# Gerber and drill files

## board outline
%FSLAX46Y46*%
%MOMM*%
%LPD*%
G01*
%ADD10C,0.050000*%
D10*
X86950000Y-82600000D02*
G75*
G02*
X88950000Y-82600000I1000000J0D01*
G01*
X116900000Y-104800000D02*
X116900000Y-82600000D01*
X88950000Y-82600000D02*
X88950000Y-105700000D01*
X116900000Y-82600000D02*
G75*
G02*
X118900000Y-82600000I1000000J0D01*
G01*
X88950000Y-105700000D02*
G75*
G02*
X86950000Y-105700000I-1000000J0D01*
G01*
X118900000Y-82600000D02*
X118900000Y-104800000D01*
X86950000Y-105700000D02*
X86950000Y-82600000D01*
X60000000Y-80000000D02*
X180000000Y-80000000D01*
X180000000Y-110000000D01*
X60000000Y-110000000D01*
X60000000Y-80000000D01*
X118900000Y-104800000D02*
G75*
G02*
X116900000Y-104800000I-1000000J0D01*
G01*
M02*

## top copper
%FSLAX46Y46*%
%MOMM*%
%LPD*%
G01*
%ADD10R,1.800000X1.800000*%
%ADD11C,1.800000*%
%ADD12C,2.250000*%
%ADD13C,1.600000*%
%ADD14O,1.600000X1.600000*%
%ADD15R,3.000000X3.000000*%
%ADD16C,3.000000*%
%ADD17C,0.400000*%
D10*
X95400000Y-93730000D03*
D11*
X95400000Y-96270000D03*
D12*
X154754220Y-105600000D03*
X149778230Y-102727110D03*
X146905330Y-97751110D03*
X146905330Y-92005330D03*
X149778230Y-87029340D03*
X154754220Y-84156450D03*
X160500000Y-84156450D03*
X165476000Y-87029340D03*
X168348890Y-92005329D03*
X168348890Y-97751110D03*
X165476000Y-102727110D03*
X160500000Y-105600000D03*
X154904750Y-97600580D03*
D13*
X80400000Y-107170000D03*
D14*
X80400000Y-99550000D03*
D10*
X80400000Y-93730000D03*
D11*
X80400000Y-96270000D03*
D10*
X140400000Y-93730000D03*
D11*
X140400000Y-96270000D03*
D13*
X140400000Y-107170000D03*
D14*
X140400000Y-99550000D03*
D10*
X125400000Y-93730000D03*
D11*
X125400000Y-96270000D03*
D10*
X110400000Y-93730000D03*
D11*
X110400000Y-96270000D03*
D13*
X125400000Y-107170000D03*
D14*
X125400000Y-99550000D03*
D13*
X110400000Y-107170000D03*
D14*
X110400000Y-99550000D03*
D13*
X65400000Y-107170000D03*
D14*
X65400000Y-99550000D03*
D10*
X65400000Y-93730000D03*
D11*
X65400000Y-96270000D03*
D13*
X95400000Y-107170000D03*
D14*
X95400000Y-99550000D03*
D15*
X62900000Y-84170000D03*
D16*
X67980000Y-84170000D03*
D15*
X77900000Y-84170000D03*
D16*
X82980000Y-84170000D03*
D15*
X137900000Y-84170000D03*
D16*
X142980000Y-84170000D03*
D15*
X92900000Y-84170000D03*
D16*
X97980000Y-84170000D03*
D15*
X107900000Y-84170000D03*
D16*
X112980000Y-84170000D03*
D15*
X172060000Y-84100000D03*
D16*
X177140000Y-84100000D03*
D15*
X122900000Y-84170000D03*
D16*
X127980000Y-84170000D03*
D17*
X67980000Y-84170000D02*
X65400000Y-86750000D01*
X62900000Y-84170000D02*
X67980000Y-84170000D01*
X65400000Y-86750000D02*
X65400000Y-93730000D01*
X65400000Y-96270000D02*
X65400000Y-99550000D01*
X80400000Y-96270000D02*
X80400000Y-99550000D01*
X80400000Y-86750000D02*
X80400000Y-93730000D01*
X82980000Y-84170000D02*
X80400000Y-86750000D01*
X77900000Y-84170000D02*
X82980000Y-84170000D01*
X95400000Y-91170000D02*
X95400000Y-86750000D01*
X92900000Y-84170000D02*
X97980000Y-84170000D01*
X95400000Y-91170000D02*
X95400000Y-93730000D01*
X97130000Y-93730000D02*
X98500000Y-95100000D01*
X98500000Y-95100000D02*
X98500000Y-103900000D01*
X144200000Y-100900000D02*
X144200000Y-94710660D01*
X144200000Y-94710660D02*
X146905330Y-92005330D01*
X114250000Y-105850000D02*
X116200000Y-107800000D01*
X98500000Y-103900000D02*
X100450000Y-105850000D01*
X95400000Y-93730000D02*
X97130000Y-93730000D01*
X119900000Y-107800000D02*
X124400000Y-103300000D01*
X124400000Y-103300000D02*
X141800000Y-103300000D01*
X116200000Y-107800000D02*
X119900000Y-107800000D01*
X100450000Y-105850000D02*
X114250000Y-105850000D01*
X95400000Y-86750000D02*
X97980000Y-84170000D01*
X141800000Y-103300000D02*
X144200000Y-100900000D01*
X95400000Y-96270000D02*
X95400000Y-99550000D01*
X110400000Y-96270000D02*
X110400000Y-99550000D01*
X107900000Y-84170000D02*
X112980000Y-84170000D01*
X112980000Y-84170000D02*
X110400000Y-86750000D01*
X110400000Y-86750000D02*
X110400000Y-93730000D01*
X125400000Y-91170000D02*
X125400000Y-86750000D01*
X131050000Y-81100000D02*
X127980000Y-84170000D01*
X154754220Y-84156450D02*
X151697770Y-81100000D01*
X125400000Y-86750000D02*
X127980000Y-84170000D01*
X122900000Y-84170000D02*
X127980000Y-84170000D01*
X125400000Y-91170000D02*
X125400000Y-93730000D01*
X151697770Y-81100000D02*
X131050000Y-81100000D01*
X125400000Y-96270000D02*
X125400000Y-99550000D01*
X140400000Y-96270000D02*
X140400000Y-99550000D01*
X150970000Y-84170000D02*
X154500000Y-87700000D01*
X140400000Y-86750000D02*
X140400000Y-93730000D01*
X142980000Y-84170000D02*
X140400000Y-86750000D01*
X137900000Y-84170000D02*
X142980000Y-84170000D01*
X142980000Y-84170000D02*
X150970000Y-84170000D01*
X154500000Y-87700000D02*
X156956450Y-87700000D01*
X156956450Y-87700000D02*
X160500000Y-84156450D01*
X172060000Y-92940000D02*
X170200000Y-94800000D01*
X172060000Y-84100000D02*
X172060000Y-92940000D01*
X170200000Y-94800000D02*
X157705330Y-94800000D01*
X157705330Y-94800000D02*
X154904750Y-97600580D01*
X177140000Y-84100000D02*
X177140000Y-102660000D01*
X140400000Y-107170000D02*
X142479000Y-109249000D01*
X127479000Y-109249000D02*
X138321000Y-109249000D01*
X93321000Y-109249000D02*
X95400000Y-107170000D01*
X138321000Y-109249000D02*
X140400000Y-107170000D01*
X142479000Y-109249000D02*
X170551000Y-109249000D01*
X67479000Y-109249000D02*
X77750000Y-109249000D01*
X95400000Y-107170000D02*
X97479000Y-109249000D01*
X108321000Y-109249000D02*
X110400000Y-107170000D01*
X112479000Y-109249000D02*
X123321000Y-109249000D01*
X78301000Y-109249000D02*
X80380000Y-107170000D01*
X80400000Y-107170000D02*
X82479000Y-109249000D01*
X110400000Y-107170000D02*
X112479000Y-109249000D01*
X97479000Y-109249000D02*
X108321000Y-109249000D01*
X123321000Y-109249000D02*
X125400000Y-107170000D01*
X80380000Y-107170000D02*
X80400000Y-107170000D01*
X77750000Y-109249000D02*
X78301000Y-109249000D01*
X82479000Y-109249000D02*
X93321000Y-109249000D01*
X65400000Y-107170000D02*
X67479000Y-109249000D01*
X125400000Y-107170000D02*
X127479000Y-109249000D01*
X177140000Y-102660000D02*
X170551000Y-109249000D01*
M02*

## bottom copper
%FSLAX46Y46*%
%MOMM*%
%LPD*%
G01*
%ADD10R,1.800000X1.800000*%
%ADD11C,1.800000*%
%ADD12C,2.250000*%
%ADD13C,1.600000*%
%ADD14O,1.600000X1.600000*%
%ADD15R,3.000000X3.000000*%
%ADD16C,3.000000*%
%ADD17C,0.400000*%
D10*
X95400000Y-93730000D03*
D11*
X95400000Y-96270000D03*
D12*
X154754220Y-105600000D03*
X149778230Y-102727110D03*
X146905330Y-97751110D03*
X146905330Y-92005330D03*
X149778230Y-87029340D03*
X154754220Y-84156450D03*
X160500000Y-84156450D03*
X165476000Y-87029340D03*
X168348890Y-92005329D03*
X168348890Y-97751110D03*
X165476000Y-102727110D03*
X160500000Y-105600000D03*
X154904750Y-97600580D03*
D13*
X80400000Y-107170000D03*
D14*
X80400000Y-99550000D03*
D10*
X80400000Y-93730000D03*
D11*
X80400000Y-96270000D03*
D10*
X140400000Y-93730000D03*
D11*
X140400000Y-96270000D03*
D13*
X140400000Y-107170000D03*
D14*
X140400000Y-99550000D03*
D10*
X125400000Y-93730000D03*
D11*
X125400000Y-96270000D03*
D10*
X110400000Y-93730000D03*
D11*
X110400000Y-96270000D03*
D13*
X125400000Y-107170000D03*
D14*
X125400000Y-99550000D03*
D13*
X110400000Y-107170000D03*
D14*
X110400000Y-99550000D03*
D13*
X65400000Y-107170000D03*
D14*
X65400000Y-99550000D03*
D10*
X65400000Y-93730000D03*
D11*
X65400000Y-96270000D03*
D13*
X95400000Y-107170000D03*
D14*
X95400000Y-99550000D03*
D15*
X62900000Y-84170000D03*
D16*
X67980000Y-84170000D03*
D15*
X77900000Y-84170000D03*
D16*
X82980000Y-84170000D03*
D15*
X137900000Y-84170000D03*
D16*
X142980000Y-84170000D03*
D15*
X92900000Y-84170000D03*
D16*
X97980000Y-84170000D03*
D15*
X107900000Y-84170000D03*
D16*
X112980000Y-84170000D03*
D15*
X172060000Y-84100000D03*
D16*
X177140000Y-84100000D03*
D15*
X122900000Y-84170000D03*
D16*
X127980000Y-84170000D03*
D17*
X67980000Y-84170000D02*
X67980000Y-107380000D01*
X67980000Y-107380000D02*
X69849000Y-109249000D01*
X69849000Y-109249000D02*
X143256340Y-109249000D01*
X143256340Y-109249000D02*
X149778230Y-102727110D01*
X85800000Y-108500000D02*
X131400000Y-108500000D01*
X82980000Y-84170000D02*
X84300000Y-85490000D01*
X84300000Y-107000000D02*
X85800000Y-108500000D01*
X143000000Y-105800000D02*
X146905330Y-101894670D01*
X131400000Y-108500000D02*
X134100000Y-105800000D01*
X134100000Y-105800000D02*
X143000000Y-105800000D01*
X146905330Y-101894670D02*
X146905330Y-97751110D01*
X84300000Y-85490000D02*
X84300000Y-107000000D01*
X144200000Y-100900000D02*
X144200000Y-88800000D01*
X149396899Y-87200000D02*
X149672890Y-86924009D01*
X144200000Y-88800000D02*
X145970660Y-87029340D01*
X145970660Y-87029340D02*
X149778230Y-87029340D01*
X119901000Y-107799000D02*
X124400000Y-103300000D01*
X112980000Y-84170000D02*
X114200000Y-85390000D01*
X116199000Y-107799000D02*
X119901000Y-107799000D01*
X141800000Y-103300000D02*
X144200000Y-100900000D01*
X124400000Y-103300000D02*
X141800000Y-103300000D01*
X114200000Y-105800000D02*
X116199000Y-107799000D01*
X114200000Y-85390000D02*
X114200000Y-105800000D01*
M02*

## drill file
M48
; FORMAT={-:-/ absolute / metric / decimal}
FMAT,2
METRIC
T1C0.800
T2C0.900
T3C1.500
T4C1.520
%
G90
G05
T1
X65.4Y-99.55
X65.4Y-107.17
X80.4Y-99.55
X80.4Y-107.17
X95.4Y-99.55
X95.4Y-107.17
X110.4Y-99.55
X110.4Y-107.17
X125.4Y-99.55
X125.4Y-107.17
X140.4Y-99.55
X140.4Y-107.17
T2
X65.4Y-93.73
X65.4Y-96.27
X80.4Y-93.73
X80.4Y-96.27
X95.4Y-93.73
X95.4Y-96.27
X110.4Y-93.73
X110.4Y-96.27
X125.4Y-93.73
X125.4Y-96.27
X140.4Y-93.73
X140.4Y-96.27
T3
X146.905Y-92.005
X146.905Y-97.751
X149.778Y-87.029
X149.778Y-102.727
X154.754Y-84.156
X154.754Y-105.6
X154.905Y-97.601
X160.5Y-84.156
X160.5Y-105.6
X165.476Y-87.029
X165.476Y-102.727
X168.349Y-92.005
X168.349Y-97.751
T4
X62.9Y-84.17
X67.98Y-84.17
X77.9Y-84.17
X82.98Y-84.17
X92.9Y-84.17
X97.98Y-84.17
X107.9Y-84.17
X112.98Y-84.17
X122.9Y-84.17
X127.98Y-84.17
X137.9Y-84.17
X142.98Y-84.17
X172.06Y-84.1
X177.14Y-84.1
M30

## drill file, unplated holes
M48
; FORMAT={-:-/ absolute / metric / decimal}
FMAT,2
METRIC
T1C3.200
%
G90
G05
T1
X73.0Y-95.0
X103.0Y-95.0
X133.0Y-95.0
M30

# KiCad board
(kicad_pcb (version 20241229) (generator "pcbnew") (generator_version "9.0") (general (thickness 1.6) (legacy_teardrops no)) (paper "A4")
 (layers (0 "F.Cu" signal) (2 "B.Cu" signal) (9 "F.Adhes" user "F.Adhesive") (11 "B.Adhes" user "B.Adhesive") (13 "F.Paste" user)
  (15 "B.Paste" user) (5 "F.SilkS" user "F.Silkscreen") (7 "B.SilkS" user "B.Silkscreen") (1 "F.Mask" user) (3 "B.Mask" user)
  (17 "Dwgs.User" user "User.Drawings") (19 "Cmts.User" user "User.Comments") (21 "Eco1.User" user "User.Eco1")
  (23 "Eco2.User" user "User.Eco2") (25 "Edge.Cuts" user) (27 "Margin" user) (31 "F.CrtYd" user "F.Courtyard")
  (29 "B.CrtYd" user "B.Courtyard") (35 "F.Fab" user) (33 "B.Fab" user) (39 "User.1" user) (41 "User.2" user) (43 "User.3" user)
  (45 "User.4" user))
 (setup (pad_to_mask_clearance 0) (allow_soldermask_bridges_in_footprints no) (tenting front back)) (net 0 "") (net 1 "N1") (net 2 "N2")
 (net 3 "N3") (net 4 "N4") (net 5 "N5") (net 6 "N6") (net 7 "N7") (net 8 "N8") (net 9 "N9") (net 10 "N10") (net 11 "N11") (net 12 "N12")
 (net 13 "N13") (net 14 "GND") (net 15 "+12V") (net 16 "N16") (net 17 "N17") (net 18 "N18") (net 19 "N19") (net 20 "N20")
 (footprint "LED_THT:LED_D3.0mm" (layer "F.Cu") (at 95.4 93.73 -90)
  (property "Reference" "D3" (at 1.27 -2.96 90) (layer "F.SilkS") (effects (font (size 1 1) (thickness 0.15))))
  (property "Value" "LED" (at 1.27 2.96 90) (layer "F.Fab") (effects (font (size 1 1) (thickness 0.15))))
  (pad "1" thru_hole rect (at 0 0 270) (size 1.8 1.8) (drill 0.9) (layers "*.Cu" "*.Mask") (remove_unused_layers no) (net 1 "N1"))
  (pad "2" thru_hole circle (at 2.54 0 270) (size 1.8 1.8) (drill 0.9) (layers "*.Cu" "*.Mask") (remove_unused_layers no) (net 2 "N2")))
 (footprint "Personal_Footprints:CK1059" (layer "F.Cu") (at 154.75422 105.6)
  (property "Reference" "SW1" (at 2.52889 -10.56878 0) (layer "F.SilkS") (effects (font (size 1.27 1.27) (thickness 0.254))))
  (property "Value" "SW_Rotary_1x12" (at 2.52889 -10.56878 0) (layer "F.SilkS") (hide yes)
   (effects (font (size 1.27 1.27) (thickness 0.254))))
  (pad "1" thru_hole circle (at 0 0) (size 2.25 2.25) (drill 1.5) (layers "*.Cu" "*.Mask") (remove_unused_layers no) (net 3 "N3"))
  (pad "2" thru_hole circle (at -4.97599 -2.87289) (size 2.25 2.25) (drill 1.5) (layers "*.Cu" "*.Mask") (remove_unused_layers no)
   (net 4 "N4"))
  (pad "3" thru_hole circle (at -7.84889 -7.84889) (size 2.25 2.25) (drill 1.5) (layers "*.Cu" "*.Mask") (remove_unused_layers no)
   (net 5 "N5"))
  (pad "4" thru_hole circle (at -7.84889 -13.59467) (size 2.25 2.25) (drill 1.5) (layers "*.Cu" "*.Mask") (remove_unused_layers no)
   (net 1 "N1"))
  (pad "5" thru_hole circle (at -4.97599 -18.57066) (size 2.25 2.25) (drill 1.5) (layers "*.Cu" "*.Mask") (remove_unused_layers no)
   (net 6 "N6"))
  (pad "6" thru_hole circle (at 0 -21.44355) (size 2.25 2.25) (drill 1.5) (layers "*.Cu" "*.Mask") (remove_unused_layers no) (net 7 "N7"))
  (pad "7" thru_hole circle (at 5.74578 -21.44355) (size 2.25 2.25) (drill 1.5) (layers "*.Cu" "*.Mask") (remove_unused_layers no)
   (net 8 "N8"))
  (pad "8" thru_hole circle (at 10.72178 -18.57066) (size 2.25 2.25) (drill 1.5) (layers "*.Cu" "*.Mask") (remove_unused_layers no)
   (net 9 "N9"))
  (pad "9" thru_hole circle (at 13.59467 -13.594671) (size 2.25 2.25) (drill 1.5) (layers "*.Cu" "*.Mask") (remove_unused_layers no)
   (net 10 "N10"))
  (pad "10" thru_hole circle (at 13.59467 -7.84889) (size 2.25 2.25) (drill 1.5) (layers "*.Cu" "*.Mask") (remove_unused_layers no)
   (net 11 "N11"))
  (pad "11" thru_hole circle (at 10.72178 -2.87289) (size 2.25 2.25) (drill 1.5) (layers "*.Cu" "*.Mask") (remove_unused_layers no)
   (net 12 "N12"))
  (pad "12" thru_hole circle (at 5.74578 0) (size 2.25 2.25) (drill 1.5) (layers "*.Cu" "*.Mask") (remove_unused_layers no) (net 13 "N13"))
  (pad "13" thru_hole circle (at 0.15053 -7.99942) (size 2.25 2.25) (drill 1.5) (layers "*.Cu" "*.Mask") (remove_unused_layers no)
   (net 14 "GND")))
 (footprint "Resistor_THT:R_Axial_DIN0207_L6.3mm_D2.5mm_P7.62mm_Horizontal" (layer "F.Cu") (at 80.4 107.17 90)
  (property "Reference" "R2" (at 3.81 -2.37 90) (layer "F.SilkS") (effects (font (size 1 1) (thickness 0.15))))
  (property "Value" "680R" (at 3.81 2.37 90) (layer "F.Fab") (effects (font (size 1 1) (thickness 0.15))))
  (pad "1" thru_hole circle (at 0 0 90) (size 1.6 1.6) (drill 0.8) (layers "*.Cu" "*.Mask") (remove_unused_layers no) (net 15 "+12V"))
  (pad "2" thru_hole oval (at 7.62 0 90) (size 1.6 1.6) (drill 0.8) (layers "*.Cu" "*.Mask") (remove_unused_layers no) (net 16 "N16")))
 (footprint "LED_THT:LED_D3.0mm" (layer "F.Cu") (at 80.4 93.73 -90)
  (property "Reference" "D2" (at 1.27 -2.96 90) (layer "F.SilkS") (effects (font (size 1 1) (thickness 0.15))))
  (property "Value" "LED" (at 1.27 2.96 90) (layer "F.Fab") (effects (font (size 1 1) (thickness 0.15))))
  (pad "1" thru_hole rect (at 0 0 270) (size 1.8 1.8) (drill 0.9) (layers "*.Cu" "*.Mask") (remove_unused_layers no) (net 5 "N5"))
  (pad "2" thru_hole circle (at 2.54 0 270) (size 1.8 1.8) (drill 0.9) (layers "*.Cu" "*.Mask") (remove_unused_layers no) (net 16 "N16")))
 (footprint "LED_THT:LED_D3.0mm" (layer "F.Cu") (at 140.4 93.73 -90)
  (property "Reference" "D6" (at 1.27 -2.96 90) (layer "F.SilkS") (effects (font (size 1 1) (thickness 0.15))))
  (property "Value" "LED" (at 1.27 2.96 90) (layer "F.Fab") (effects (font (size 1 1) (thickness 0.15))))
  (pad "1" thru_hole rect (at 0 0 270) (size 1.8 1.8) (drill 0.9) (layers "*.Cu" "*.Mask") (remove_unused_layers no) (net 8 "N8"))
  (pad "2" thru_hole circle (at 2.54 0 270) (size 1.8 1.8) (drill 0.9) (layers "*.Cu" "*.Mask") (remove_unused_layers no) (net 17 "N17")))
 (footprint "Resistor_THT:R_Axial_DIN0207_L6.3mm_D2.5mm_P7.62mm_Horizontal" (layer "F.Cu") (at 140.4 107.17 90)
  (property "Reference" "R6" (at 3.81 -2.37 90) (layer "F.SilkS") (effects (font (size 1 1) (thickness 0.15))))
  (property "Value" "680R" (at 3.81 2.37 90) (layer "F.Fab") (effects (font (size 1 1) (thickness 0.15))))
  (pad "1" thru_hole circle (at 0 0 90) (size 1.6 1.6) (drill 0.8) (layers "*.Cu" "*.Mask") (remove_unused_layers no) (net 15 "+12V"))
  (pad "2" thru_hole oval (at 7.62 0 90) (size 1.6 1.6) (drill 0.8) (layers "*.Cu" "*.Mask") (remove_unused_layers no) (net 17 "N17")))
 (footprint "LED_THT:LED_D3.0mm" (layer "F.Cu") (at 125.4 93.73 -90)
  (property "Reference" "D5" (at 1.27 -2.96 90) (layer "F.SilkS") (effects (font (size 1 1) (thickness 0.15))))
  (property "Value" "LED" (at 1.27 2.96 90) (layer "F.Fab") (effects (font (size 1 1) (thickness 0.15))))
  (pad "1" thru_hole rect (at 0 0 270) (size 1.8 1.8) (drill 0.9) (layers "*.Cu" "*.Mask") (remove_unused_layers no) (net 7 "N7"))
  (pad "2" thru_hole circle (at 2.54 0 270) (size 1.8 1.8) (drill 0.9) (layers "*.Cu" "*.Mask") (remove_unused_layers no) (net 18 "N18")))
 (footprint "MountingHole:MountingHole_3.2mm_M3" (layer "F.Cu") (at 103 95)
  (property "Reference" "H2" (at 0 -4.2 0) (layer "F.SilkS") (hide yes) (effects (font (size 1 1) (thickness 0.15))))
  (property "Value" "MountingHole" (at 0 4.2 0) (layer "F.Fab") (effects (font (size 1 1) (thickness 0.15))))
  (pad "" np_thru_hole circle (at 0 0) (size 3.2 3.2) (drill 3.2) (layers "*.Cu" "*.Mask")))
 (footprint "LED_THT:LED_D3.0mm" (layer "F.Cu") (at 110.4 93.73 -90)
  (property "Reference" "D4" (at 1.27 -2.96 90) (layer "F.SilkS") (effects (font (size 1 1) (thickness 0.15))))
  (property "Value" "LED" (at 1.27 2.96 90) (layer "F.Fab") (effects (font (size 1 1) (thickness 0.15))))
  (pad "1" thru_hole rect (at 0 0 270) (size 1.8 1.8) (drill 0.9) (layers "*.Cu" "*.Mask") (remove_unused_layers no) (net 6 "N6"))
  (pad "2" thru_hole circle (at 2.54 0 270) (size 1.8 1.8) (drill 0.9) (layers "*.Cu" "*.Mask") (remove_unused_layers no) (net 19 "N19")))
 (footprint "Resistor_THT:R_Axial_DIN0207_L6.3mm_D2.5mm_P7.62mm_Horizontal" (layer "F.Cu") (at 125.4 107.17 90)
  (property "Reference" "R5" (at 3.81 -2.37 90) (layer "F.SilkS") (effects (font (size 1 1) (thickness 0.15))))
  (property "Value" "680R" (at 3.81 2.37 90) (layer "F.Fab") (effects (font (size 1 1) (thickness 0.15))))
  (pad "1" thru_hole circle (at 0 0 90) (size 1.6 1.6) (drill 0.8) (layers "*.Cu" "*.Mask") (remove_unused_layers no) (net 15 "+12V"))
  (pad "2" thru_hole oval (at 7.62 0 90) (size 1.6 1.6) (drill 0.8) (layers "*.Cu" "*.Mask") (remove_unused_layers no) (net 18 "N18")))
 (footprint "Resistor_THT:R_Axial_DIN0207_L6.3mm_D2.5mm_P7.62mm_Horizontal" (layer "F.Cu") (at 110.4 107.17 90)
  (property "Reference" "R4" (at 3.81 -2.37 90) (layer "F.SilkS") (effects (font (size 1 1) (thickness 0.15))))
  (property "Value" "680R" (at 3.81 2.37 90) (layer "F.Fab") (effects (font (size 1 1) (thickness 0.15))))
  (pad "1" thru_hole circle (at 0 0 90) (size 1.6 1.6) (drill 0.8) (layers "*.Cu" "*.Mask") (remove_unused_layers no) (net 15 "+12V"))
  (pad "2" thru_hole oval (at 7.62 0 90) (size 1.6 1.6) (drill 0.8) (layers "*.Cu" "*.Mask") (remove_unused_layers no) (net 19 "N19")))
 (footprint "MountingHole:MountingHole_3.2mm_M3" (layer "F.Cu") (at 73 95)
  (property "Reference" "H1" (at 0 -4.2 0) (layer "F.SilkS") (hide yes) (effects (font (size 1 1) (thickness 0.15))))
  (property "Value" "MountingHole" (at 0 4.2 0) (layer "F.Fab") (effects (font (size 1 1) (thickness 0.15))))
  (pad "" np_thru_hole circle (at 0 0) (size 3.2 3.2) (drill 3.2) (layers "*.Cu" "*.Mask")))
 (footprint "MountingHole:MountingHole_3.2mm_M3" (layer "F.Cu") (at 133 95)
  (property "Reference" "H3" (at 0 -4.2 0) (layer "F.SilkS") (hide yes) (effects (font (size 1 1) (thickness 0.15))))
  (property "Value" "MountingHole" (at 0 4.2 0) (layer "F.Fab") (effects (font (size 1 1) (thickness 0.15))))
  (pad "" np_thru_hole circle (at 0 0) (size 3.2 3.2) (drill 3.2) (layers "*.Cu" "*.Mask")))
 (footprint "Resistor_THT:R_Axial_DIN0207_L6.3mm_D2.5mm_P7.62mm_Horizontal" (layer "F.Cu") (at 65.4 107.17 90)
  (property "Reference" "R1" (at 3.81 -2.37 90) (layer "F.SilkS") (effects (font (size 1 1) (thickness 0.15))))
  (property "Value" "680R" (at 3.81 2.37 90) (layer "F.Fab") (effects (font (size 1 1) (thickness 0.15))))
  (pad "1" thru_hole circle (at 0 0 90) (size 1.6 1.6) (drill 0.8) (layers "*.Cu" "*.Mask") (remove_unused_layers no) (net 15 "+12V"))
  (pad "2" thru_hole oval (at 7.62 0 90) (size 1.6 1.6) (drill 0.8) (layers "*.Cu" "*.Mask") (remove_unused_layers no) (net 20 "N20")))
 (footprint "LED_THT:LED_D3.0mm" (layer "F.Cu") (at 65.4 93.73 -90)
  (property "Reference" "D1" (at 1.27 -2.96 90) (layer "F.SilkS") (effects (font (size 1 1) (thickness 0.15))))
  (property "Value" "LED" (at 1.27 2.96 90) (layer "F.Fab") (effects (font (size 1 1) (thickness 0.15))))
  (pad "1" thru_hole rect (at 0 0 270) (size 1.8 1.8) (drill 0.9) (layers "*.Cu" "*.Mask") (remove_unused_layers no) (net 4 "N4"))
  (pad "2" thru_hole circle (at 2.54 0 270) (size 1.8 1.8) (drill 0.9) (layers "*.Cu" "*.Mask") (remove_unused_layers no) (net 20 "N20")))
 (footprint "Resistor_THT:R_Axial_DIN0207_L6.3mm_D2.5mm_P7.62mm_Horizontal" (layer "F.Cu") (at 95.4 107.17 90)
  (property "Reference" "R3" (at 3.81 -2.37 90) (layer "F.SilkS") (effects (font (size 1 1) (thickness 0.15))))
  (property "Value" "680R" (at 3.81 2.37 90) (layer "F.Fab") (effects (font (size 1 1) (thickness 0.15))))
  (pad "1" thru_hole circle (at 0 0 90) (size 1.6 1.6) (drill 0.8) (layers "*.Cu" "*.Mask") (remove_unused_layers no) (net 15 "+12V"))
  (pad "2" thru_hole oval (at 7.62 0 90) (size 1.6 1.6) (drill 0.8) (layers "*.Cu" "*.Mask") (remove_unused_layers no) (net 2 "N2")))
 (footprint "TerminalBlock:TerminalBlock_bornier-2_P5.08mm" (layer "B.Cu") (at 62.9 84.17)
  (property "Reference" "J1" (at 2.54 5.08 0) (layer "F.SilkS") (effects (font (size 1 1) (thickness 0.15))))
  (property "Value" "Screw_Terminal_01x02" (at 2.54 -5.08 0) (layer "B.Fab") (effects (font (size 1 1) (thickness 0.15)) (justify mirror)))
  (pad "1" thru_hole rect (at 0 0) (size 3 3) (drill 1.52) (layers "*.Cu" "*.Mask") (remove_unused_layers no) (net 4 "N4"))
  (pad "2" thru_hole circle (at 5.08 0) (size 3 3) (drill 1.52) (layers "*.Cu" "*.Mask") (remove_unused_layers no) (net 4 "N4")))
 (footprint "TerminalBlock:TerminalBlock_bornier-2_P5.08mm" (layer "B.Cu") (at 77.9 84.17)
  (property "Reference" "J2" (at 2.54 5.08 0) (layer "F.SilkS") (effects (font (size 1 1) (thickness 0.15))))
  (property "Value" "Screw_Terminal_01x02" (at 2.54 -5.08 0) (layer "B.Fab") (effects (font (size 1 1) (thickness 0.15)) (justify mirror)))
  (pad "1" thru_hole rect (at 0 0) (size 3 3) (drill 1.52) (layers "*.Cu" "*.Mask") (remove_unused_layers no) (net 5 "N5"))
  (pad "2" thru_hole circle (at 5.08 0) (size 3 3) (drill 1.52) (layers "*.Cu" "*.Mask") (remove_unused_layers no) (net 5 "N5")))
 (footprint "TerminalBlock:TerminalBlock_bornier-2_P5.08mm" (layer "B.Cu") (at 137.9 84.17)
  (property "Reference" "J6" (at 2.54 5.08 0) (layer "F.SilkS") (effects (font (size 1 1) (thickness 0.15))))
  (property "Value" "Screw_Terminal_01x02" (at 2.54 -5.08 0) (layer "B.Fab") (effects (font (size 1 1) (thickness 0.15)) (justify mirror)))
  (pad "1" thru_hole rect (at 0 0) (size 3 3) (drill 1.52) (layers "*.Cu" "*.Mask") (remove_unused_layers no) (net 8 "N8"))
  (pad "2" thru_hole circle (at 5.08 0) (size 3 3) (drill 1.52) (layers "*.Cu" "*.Mask") (remove_unused_layers no) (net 8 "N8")))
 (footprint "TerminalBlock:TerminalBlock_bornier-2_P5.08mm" (layer "B.Cu") (at 92.9 84.17)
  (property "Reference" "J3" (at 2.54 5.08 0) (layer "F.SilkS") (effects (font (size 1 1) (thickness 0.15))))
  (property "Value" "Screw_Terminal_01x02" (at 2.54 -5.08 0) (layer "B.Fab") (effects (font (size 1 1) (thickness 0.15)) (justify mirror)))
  (pad "1" thru_hole rect (at 0 0) (size 3 3) (drill 1.52) (layers "*.Cu" "*.Mask") (remove_unused_layers no) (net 1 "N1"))
  (pad "2" thru_hole circle (at 5.08 0) (size 3 3) (drill 1.52) (layers "*.Cu" "*.Mask") (remove_unused_layers no) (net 1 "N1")))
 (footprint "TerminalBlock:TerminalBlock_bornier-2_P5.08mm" (layer "B.Cu") (at 107.9 84.17)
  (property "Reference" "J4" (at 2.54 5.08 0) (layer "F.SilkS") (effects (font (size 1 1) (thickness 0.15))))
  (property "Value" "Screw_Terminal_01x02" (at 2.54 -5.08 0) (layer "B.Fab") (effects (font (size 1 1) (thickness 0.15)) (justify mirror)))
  (pad "1" thru_hole rect (at 0 0) (size 3 3) (drill 1.52) (layers "*.Cu" "*.Mask") (remove_unused_layers no) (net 6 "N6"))
  (pad "2" thru_hole circle (at 5.08 0) (size 3 3) (drill 1.52) (layers "*.Cu" "*.Mask") (remove_unused_layers no) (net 6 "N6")))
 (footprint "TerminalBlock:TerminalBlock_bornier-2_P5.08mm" (layer "B.Cu") (at 172.06 84.1)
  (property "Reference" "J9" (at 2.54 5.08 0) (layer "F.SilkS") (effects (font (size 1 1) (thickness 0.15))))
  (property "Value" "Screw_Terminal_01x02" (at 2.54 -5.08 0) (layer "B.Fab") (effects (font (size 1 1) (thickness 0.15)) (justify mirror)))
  (pad "1" thru_hole rect (at 0 0) (size 3 3) (drill 1.52) (layers "*.Cu" "*.Mask") (remove_unused_layers no) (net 14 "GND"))
  (pad "2" thru_hole circle (at 5.08 0) (size 3 3) (drill 1.52) (layers "*.Cu" "*.Mask") (remove_unused_layers no) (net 15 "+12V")))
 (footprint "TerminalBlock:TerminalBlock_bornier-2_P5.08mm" (layer "B.Cu") (at 122.9 84.17)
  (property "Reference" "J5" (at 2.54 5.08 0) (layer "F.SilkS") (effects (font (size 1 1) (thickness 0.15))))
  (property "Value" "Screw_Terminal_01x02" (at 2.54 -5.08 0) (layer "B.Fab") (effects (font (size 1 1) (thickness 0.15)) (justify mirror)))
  (pad "1" thru_hole rect (at 0 0) (size 3 3) (drill 1.52) (layers "*.Cu" "*.Mask") (remove_unused_layers no) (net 7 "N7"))
  (pad "2" thru_hole circle (at 5.08 0) (size 3 3) (drill 1.52) (layers "*.Cu" "*.Mask") (remove_unused_layers no) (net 7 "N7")))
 (gr_arc (start 86.95 82.6) (mid 87.95 81.6) (end 88.95 82.6) (stroke (width 0.05) (type default)) (layer "Edge.Cuts"))
 (gr_line (start 116.9 104.8) (end 116.9 82.6) (stroke (width 0.05) (type default)) (layer "Edge.Cuts"))
 (gr_line (start 88.95 82.6) (end 88.95 105.7) (stroke (width 0.05) (type default)) (layer "Edge.Cuts"))
 (gr_arc (start 116.9 82.6) (mid 117.9 81.6) (end 118.9 82.6) (stroke (width 0.05) (type default)) (layer "Edge.Cuts"))
 (gr_arc (start 88.95 105.7) (mid 87.95 106.7) (end 86.95 105.7) (stroke (width 0.05) (type default)) (layer "Edge.Cuts"))
 (gr_line (start 118.9 82.6) (end 118.9 104.8) (stroke (width 0.05) (type default)) (layer "Edge.Cuts"))
 (gr_line (start 86.95 105.7) (end 86.95 82.6) (stroke (width 0.05) (type default)) (layer "Edge.Cuts"))
 (gr_rect (start 60 80) (end 180 110) (stroke (width 0.05) (type solid)) (fill no) (layer "Edge.Cuts"))
 (gr_arc (start 118.9 104.8) (mid 117.9 105.8) (end 116.9 104.8) (stroke (width 0.05) (type default)) (layer "Edge.Cuts"))
 (segment (start 67.98 84.17) (end 65.4 86.75) (width 0.4) (layer "F.Cu") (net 4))
 (segment (start 62.9 84.17) (end 67.98 84.17) (width 0.4) (layer "F.Cu") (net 4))
 (segment (start 65.4 86.75) (end 65.4 93.73) (width 0.4) (layer "F.Cu") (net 4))
 (segment (start 67.98 84.17) (end 67.98 107.38) (width 0.4) (layer "B.Cu") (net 4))
 (segment (start 67.98 107.38) (end 69.849 109.249) (width 0.4) (layer "B.Cu") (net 4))
 (segment (start 69.849 109.249) (end 143.25634 109.249) (width 0.4) (layer "B.Cu") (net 4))
 (segment (start 143.25634 109.249) (end 149.77823 102.72711) (width 0.4) (layer "B.Cu") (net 4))
 (segment (start 65.4 96.27) (end 65.4 99.55) (width 0.4) (layer "F.Cu") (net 20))
 (segment (start 80.4 96.27) (end 80.4 99.55) (width 0.4) (layer "F.Cu") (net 16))
 (segment (start 80.4 86.75) (end 80.4 93.73) (width 0.4) (layer "F.Cu") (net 5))
 (segment (start 82.98 84.17) (end 80.4 86.75) (width 0.4) (layer "F.Cu") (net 5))
 (segment (start 77.9 84.17) (end 82.98 84.17) (width 0.4) (layer "F.Cu") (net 5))
 (segment (start 85.8 108.5) (end 131.4 108.5) (width 0.4) (layer "B.Cu") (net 5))
 (segment (start 82.98 84.17) (end 84.3 85.49) (width 0.4) (layer "B.Cu") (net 5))
 (segment (start 84.3 107) (end 85.8 108.5) (width 0.4) (layer "B.Cu") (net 5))
 (segment (start 143 105.8) (end 146.90533 101.89467) (width 0.4) (layer "B.Cu") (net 5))
 (segment (start 131.4 108.5) (end 134.1 105.8) (width 0.4) (layer "B.Cu") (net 5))
 (segment (start 134.1 105.8) (end 143 105.8) (width 0.4) (layer "B.Cu") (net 5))
 (segment (start 146.90533 101.89467) (end 146.90533 97.75111) (width 0.4) (layer "B.Cu") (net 5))
 (segment (start 84.3 85.49) (end 84.3 107) (width 0.4) (layer "B.Cu") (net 5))
 (segment (start 95.4 91.17) (end 95.4 86.75) (width 0.4) (layer "F.Cu") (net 1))
 (segment (start 92.9 84.17) (end 97.98 84.17) (width 0.4) (layer "F.Cu") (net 1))
 (segment (start 95.4 91.17) (end 95.4 93.73) (width 0.4) (layer "F.Cu") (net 1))
 (segment (start 97.13 93.73) (end 98.5 95.1) (width 0.4) (layer "F.Cu") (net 1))
 (segment (start 98.5 95.1) (end 98.5 103.9) (width 0.4) (layer "F.Cu") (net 1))
 (segment (start 144.2 100.9) (end 144.2 94.71066) (width 0.4) (layer "F.Cu") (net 1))
 (segment (start 144.2 94.71066) (end 146.90533 92.00533) (width 0.4) (layer "F.Cu") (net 1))
 (segment (start 114.25 105.85) (end 116.2 107.8) (width 0.4) (layer "F.Cu") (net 1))
 (segment (start 98.5 103.9) (end 100.45 105.85) (width 0.4) (layer "F.Cu") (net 1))
 (segment (start 95.4 93.73) (end 97.13 93.73) (width 0.4) (layer "F.Cu") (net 1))
 (segment (start 119.9 107.8) (end 124.4 103.3) (width 0.4) (layer "F.Cu") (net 1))
 (segment (start 124.4 103.3) (end 141.8 103.3) (width 0.4) (layer "F.Cu") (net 1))
 (segment (start 116.2 107.8) (end 119.9 107.8) (width 0.4) (layer "F.Cu") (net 1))
 (segment (start 100.45 105.85) (end 114.25 105.85) (width 0.4) (layer "F.Cu") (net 1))
 (segment (start 95.4 86.75) (end 97.98 84.17) (width 0.4) (layer "F.Cu") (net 1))
 (segment (start 141.8 103.3) (end 144.2 100.9) (width 0.4) (layer "F.Cu") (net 1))
 (segment (start 95.4 96.27) (end 95.4 99.55) (width 0.4) (layer "F.Cu") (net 2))
 (segment (start 110.4 96.27) (end 110.4 99.55) (width 0.4) (layer "F.Cu") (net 19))
 (segment (start 107.9 84.17) (end 112.98 84.17) (width 0.4) (layer "F.Cu") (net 6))
 (segment (start 112.98 84.17) (end 110.4 86.75) (width 0.4) (layer "F.Cu") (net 6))
 (segment (start 110.4 86.75) (end 110.4 93.73) (width 0.4) (layer "F.Cu") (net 6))
 (segment (start 144.2 100.9) (end 144.2 88.8) (width 0.4) (layer "B.Cu") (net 6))
 (segment (start 149.396899 87.2) (end 149.67289 86.924009) (width 0.4) (layer "B.Cu") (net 6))
 (segment (start 144.2 88.8) (end 145.97066 87.02934) (width 0.4) (layer "B.Cu") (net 6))
 (segment (start 145.97066 87.02934) (end 149.77823 87.02934) (width 0.4) (layer "B.Cu") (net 6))
 (segment (start 119.901 107.799) (end 124.4 103.3) (width 0.4) (layer "B.Cu") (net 6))
 (segment (start 112.98 84.17) (end 114.2 85.39) (width 0.4) (layer "B.Cu") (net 6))
 (segment (start 116.199 107.799) (end 119.901 107.799) (width 0.4) (layer "B.Cu") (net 6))
 (segment (start 141.8 103.3) (end 144.2 100.9) (width 0.4) (layer "B.Cu") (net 6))
 (segment (start 124.4 103.3) (end 141.8 103.3) (width 0.4) (layer "B.Cu") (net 6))
 (segment (start 114.2 105.8) (end 116.199 107.799) (width 0.4) (layer "B.Cu") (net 6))
 (segment (start 114.2 85.39) (end 114.2 105.8) (width 0.4) (layer "B.Cu") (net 6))
 (segment (start 125.4 91.17) (end 125.4 86.75) (width 0.4) (layer "F.Cu") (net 7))
 (segment (start 131.05 81.1) (end 127.98 84.17) (width 0.4) (layer "F.Cu") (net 7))
 (segment (start 154.75422 84.15645) (end 151.69777 81.1) (width 0.4) (layer "F.Cu") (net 7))
 (segment (start 125.4 86.75) (end 127.98 84.17) (width 0.4) (layer "F.Cu") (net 7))
 (segment (start 122.9 84.17) (end 127.98 84.17) (width 0.4) (layer "F.Cu") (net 7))
 (segment (start 125.4 91.17) (end 125.4 93.73) (width 0.4) (layer "F.Cu") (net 7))
 (segment (start 151.69777 81.1) (end 131.05 81.1) (width 0.4) (layer "F.Cu") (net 7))
 (segment (start 125.4 96.27) (end 125.4 99.55) (width 0.4) (layer "F.Cu") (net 18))
 (segment (start 140.4 96.27) (end 140.4 99.55) (width 0.4) (layer "F.Cu") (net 17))
 (segment (start 150.97 84.17) (end 154.5 87.7) (width 0.4) (layer "F.Cu") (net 8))
 (segment (start 140.4 86.75) (end 140.4 93.73) (width 0.4) (layer "F.Cu") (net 8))
 (segment (start 142.98 84.17) (end 140.4 86.75) (width 0.4) (layer "F.Cu") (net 8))
 (segment (start 137.9 84.17) (end 142.98 84.17) (width 0.4) (layer "F.Cu") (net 8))
 (segment (start 142.98 84.17) (end 150.97 84.17) (width 0.4) (layer "F.Cu") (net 8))
 (segment (start 154.5 87.7) (end 156.95645 87.7) (width 0.4) (layer "F.Cu") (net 8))
 (segment (start 156.95645 87.7) (end 160.5 84.15645) (width 0.4) (layer "F.Cu") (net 8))
 (segment (start 172.06 92.94) (end 170.2 94.8) (width 0.4) (layer "F.Cu") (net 14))
 (segment (start 172.06 84.1) (end 172.06 92.94) (width 0.4) (layer "F.Cu") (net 14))
 (segment (start 170.2 94.8) (end 157.70533 94.8) (width 0.4) (layer "F.Cu") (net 14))
 (segment (start 157.70533 94.8) (end 154.90475 97.60058) (width 0.4) (layer "F.Cu") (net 14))
 (segment (start 177.14 84.1) (end 177.14 102.66) (width 0.4) (layer "F.Cu") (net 15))
 (segment (start 140.4 107.17) (end 142.479 109.249) (width 0.4) (layer "F.Cu") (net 15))
 (segment (start 127.479 109.249) (end 138.321 109.249) (width 0.4) (layer "F.Cu") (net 15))
 (segment (start 93.321 109.249) (end 95.4 107.17) (width 0.4) (layer "F.Cu") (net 15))
 (segment (start 138.321 109.249) (end 140.4 107.17) (width 0.4) (layer "F.Cu") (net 15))
 (segment (start 142.479 109.249) (end 170.551 109.249) (width 0.4) (layer "F.Cu") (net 15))
 (segment (start 67.479 109.249) (end 77.75 109.249) (width 0.4) (layer "F.Cu") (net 15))
 (segment (start 95.4 107.17) (end 97.479 109.249) (width 0.4) (layer "F.Cu") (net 15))
 (segment (start 108.321 109.249) (end 110.4 107.17) (width 0.4) (layer "F.Cu") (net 15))
 (segment (start 112.479 109.249) (end 123.321 109.249) (width 0.4) (layer "F.Cu") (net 15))
 (segment (start 78.301 109.249) (end 80.38 107.17) (width 0.4) (layer "F.Cu") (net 15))
 (segment (start 80.4 107.17) (end 82.479 109.249) (width 0.4) (layer "F.Cu") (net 15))
 (segment (start 110.4 107.17) (end 112.479 109.249) (width 0.4) (layer "F.Cu") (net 15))
 (segment (start 97.479 109.249) (end 108.321 109.249) (width 0.4) (layer "F.Cu") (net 15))
 (segment (start 123.321 109.249) (end 125.4 107.17) (width 0.4) (layer "F.Cu") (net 15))
 (segment (start 80.38 107.17) (end 80.4 107.17) (width 0.4) (layer "F.Cu") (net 15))
 (segment (start 77.75 109.249) (end 78.301 109.249) (width 0.4) (layer "F.Cu") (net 15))
 (segment (start 82.479 109.249) (end 93.321 109.249) (width 0.4) (layer "F.Cu") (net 15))
 (segment (start 65.4 107.17) (end 67.479 109.249) (width 0.4) (layer "F.Cu") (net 15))
 (segment (start 125.4 107.17) (end 127.479 109.249) (width 0.4) (layer "F.Cu") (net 15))
 (segment (start 177.14 102.66) (end 170.551 109.249) (width 0.4) (layer "F.Cu") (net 15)))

